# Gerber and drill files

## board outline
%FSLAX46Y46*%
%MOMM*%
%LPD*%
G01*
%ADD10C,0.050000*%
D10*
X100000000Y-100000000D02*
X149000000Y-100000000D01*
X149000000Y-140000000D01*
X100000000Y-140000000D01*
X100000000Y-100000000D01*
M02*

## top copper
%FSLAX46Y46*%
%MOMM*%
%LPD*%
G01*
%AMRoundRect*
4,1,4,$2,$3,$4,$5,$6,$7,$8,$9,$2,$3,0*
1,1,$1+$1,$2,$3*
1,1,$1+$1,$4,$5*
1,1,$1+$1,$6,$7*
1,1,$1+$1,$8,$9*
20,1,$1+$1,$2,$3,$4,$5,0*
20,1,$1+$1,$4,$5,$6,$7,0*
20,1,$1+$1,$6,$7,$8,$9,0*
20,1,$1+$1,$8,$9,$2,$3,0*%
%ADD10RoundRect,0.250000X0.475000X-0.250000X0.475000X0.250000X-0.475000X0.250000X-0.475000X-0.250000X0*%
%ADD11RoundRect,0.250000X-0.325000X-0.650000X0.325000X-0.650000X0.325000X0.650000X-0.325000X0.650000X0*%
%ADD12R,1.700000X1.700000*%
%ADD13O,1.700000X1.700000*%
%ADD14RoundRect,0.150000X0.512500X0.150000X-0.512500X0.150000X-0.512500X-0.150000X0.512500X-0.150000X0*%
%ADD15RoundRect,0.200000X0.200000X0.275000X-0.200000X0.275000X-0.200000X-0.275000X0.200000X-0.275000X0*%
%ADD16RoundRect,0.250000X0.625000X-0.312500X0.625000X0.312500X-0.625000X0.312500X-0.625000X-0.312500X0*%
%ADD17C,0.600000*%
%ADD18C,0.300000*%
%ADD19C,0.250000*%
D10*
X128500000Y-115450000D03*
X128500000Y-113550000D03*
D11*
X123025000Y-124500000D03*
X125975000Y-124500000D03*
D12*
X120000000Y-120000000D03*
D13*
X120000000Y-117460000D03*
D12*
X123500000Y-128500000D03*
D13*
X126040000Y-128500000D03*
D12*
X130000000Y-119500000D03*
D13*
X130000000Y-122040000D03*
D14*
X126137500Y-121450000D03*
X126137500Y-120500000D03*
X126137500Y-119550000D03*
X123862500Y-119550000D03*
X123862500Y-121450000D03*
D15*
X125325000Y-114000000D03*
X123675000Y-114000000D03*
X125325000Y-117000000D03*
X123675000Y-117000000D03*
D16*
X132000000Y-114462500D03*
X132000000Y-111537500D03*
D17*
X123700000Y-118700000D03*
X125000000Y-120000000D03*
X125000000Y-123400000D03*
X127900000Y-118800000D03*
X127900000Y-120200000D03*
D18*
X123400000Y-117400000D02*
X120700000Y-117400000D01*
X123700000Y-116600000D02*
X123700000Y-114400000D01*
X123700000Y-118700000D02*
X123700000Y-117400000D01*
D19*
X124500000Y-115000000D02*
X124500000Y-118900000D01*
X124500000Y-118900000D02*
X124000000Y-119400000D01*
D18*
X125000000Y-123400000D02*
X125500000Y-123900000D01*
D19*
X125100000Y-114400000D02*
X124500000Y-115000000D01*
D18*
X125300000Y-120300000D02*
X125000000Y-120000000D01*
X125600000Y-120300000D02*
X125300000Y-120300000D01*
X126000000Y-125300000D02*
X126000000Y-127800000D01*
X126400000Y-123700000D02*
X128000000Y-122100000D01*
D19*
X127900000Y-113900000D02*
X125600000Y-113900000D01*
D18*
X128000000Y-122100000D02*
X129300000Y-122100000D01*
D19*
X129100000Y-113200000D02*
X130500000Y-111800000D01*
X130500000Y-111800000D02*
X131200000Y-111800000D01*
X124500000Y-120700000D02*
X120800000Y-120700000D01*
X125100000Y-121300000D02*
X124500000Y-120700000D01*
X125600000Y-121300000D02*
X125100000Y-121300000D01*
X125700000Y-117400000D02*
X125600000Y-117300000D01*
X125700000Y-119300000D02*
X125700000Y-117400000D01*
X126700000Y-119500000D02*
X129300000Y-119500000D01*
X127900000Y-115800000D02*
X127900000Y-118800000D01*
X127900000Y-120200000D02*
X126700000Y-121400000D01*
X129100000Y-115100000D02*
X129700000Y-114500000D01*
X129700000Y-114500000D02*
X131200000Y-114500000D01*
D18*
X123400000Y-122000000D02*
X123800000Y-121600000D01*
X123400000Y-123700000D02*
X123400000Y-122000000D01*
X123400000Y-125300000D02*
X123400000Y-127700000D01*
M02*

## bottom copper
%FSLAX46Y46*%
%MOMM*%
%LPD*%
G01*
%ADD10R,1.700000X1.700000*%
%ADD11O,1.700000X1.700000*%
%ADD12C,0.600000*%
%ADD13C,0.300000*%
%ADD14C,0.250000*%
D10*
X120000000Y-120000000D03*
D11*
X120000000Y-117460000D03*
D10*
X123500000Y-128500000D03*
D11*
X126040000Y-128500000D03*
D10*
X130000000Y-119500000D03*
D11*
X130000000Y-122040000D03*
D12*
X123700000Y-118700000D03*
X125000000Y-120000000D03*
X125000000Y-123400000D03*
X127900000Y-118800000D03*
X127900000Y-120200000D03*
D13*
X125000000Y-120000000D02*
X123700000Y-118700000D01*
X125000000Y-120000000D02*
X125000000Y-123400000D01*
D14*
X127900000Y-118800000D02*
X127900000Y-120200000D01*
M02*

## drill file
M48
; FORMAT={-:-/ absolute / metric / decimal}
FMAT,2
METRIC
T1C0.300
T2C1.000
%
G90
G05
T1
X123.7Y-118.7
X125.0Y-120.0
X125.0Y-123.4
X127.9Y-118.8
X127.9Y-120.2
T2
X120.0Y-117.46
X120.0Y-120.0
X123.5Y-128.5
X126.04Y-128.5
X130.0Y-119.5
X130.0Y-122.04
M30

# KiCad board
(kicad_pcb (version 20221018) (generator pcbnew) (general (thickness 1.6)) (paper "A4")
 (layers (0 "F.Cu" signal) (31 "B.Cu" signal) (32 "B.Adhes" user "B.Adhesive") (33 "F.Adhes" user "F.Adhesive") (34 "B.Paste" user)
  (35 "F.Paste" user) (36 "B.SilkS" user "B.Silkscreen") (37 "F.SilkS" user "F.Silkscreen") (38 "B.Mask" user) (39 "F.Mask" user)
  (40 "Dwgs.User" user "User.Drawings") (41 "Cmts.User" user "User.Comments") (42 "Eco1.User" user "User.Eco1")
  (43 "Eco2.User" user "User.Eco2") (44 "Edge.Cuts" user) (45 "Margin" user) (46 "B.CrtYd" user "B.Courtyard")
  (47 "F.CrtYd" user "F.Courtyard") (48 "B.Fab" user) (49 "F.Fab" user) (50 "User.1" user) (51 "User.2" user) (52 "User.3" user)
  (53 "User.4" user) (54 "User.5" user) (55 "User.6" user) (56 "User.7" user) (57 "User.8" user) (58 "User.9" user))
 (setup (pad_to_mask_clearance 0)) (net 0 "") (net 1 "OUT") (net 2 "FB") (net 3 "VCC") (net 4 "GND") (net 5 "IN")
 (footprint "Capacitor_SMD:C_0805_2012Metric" (layer "F.Cu") (at 128.5 114.5 90)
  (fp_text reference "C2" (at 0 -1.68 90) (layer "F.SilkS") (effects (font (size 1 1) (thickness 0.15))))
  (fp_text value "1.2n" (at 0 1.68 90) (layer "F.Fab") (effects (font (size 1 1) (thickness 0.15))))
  (pad "1" smd roundrect (at -0.95 0 90) (size 1 1.45) (layers "F.Cu" "F.Paste" "F.Mask") (roundrect_rratio 0.25) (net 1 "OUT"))
  (pad "2" smd roundrect (at 0.95 0 90) (size 1 1.45) (layers "F.Cu" "F.Paste" "F.Mask") (roundrect_rratio 0.25) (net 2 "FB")))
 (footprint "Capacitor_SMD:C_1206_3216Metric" (layer "F.Cu") (at 124.5 124.5)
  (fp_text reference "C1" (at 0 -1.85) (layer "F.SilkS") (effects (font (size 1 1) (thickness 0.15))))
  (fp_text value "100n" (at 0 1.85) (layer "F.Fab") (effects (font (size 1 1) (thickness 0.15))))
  (pad "1" smd roundrect (at -1.475 0) (size 1.15 1.8) (layers "F.Cu" "F.Paste" "F.Mask") (roundrect_rratio 0.217391) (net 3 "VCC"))
  (pad "2" smd roundrect (at 1.475 0) (size 1.15 1.8) (layers "F.Cu" "F.Paste" "F.Mask") (roundrect_rratio 0.217391) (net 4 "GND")))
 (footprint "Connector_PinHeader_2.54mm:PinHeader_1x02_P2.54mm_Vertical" (layer "F.Cu") (at 120 120 180)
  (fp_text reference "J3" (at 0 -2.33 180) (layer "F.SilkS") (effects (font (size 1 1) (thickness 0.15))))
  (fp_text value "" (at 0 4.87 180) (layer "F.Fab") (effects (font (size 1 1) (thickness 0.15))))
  (pad "1" thru_hole rect (at 0 0 180) (size 1.7 1.7) (drill 1) (layers "*.Cu" "*.Mask") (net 1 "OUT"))
  (pad "2" thru_hole oval (at 0 2.54 180) (size 1.7 1.7) (drill 1) (layers "*.Cu" "*.Mask") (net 4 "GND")))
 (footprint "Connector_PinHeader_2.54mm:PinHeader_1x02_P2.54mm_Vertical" (layer "F.Cu") (at 123.5 128.5 90)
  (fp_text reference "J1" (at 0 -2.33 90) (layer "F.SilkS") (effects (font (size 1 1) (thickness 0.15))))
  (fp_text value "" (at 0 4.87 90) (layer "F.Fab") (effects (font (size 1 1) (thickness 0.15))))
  (pad "1" thru_hole rect (at 0 0 90) (size 1.7 1.7) (drill 1) (layers "*.Cu" "*.Mask") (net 3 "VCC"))
  (pad "2" thru_hole oval (at 0 2.54 90) (size 1.7 1.7) (drill 1) (layers "*.Cu" "*.Mask") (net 4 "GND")))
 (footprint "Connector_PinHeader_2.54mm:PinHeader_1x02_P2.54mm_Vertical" (layer "F.Cu") (at 130 119.5)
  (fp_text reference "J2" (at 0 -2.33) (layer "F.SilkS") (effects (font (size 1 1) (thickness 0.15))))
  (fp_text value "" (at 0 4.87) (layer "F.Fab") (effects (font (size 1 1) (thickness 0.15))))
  (pad "1" thru_hole rect (at 0 0) (size 1.7 1.7) (drill 1) (layers "*.Cu" "*.Mask") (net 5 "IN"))
  (pad "2" thru_hole oval (at 0 2.54) (size 1.7 1.7) (drill 1) (layers "*.Cu" "*.Mask") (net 4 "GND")))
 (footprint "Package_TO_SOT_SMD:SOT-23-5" (layer "F.Cu") (at 125 120.5 180)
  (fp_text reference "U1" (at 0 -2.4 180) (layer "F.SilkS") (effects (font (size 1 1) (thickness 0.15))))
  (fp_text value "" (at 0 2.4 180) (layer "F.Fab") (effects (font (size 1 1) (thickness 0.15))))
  (pad "1" smd roundrect (at -1.1375 -0.95 180) (size 1.325 0.6) (layers "F.Cu" "F.Paste" "F.Mask") (roundrect_rratio 0.25) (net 1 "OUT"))
  (pad "2" smd roundrect (at -1.1375 0 180) (size 1.325 0.6) (layers "F.Cu" "F.Paste" "F.Mask") (roundrect_rratio 0.25) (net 4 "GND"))
  (pad "3" smd roundrect (at -1.1375 0.95 180) (size 1.325 0.6) (layers "F.Cu" "F.Paste" "F.Mask") (roundrect_rratio 0.25) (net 5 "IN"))
  (pad "4" smd roundrect (at 1.1375 0.95 180) (size 1.325 0.6) (layers "F.Cu" "F.Paste" "F.Mask") (roundrect_rratio 0.25) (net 2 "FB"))
  (pad "5" smd roundrect (at 1.1375 -0.95 180) (size 1.325 0.6) (layers "F.Cu" "F.Paste" "F.Mask") (roundrect_rratio 0.25) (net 3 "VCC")))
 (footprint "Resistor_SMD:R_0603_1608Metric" (layer "F.Cu") (at 124.5 114 180)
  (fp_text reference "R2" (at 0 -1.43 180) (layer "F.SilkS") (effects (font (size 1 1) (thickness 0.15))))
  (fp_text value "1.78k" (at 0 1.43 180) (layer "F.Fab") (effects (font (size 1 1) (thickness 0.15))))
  (pad "1" smd roundrect (at -0.825 0 180) (size 0.8 0.95) (layers "F.Cu" "F.Paste" "F.Mask") (roundrect_rratio 0.25) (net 2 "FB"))
  (pad "2" smd roundrect (at 0.825 0 180) (size 0.8 0.95) (layers "F.Cu" "F.Paste" "F.Mask") (roundrect_rratio 0.25) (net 4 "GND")))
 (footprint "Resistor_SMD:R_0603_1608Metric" (layer "F.Cu") (at 124.5 117 180)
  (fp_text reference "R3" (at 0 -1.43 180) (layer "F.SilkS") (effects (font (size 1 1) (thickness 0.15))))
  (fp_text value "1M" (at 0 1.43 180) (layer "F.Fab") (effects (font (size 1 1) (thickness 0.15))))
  (pad "1" smd roundrect (at -0.825 0 180) (size 0.8 0.95) (layers "F.Cu" "F.Paste" "F.Mask") (roundrect_rratio 0.25) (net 5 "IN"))
  (pad "2" smd roundrect (at 0.825 0 180) (size 0.8 0.95) (layers "F.Cu" "F.Paste" "F.Mask") (roundrect_rratio 0.25) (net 4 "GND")))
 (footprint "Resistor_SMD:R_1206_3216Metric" (layer "F.Cu") (at 132 113 90)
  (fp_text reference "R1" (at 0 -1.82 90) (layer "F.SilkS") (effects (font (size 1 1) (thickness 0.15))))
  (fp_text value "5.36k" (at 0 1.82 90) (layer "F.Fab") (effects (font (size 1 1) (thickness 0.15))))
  (pad "1" smd roundrect (at -1.4625 0 90) (size 1.125 1.75) (layers "F.Cu" "F.Paste" "F.Mask") (roundrect_rratio 0.222222) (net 1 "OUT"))
  (pad "2" smd roundrect (at 1.4625 0 90) (size 1.125 1.75) (layers "F.Cu" "F.Paste" "F.Mask") (roundrect_rratio 0.222222) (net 2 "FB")))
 (gr_rect (start 100 100) (end 149 140) (stroke (width 0.05) (type default)) (fill none) (layer "Edge.Cuts"))
 (segment (start 123.4 117.4) (end 120.7 117.4) (width 0.3) (layer "F.Cu") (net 4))
 (segment (start 123.7 116.6) (end 123.7 114.4) (width 0.3) (layer "F.Cu") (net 4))
 (segment (start 123.7 118.7) (end 123.7 117.4) (width 0.3) (layer "F.Cu") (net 4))
 (segment (start 124.5 115) (end 124.5 118.9) (width 0.25) (layer "F.Cu") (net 2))
 (segment (start 124.5 118.9) (end 124 119.4) (width 0.25) (layer "F.Cu") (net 2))
 (segment (start 125 123.4) (end 125.5 123.9) (width 0.3) (layer "F.Cu") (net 4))
 (segment (start 125.1 114.4) (end 124.5 115) (width 0.25) (layer "F.Cu") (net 2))
 (segment (start 125.3 120.3) (end 125 120) (width 0.3) (layer "F.Cu") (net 4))
 (segment (start 125.6 120.3) (end 125.3 120.3) (width 0.3) (layer "F.Cu") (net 4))
 (segment (start 126 125.3) (end 126 127.8) (width 0.3) (layer "F.Cu") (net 4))
 (segment (start 126.4 123.7) (end 128 122.1) (width 0.3) (layer "F.Cu") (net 4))
 (segment (start 127.9 113.9) (end 125.6 113.9) (width 0.25) (layer "F.Cu") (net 2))
 (segment (start 128 122.1) (end 129.3 122.1) (width 0.3) (layer "F.Cu") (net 4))
 (segment (start 129.1 113.2) (end 130.5 111.8) (width 0.25) (layer "F.Cu") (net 2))
 (segment (start 130.5 111.8) (end 131.2 111.8) (width 0.25) (layer "F.Cu") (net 2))
 (via (at 123.7 118.7) (size 0.6) (drill 0.3) (layers "F.Cu" "B.Cu") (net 4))
 (via (at 125 120) (size 0.6) (drill 0.3) (layers "F.Cu" "B.Cu") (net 4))
 (via (at 125 123.4) (size 0.6) (drill 0.3) (layers "F.Cu" "B.Cu") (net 4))
 (segment (start 124.5 120.7) (end 120.8 120.7) (width 0.25) (layer "F.Cu") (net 1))
 (segment (start 125 120) (end 123.7 118.7) (width 0.3) (layer "B.Cu") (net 4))
 (segment (start 125 120) (end 125 123.4) (width 0.3) (layer "B.Cu") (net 4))
 (segment (start 125.1 121.3) (end 124.5 120.7) (width 0.25) (layer "F.Cu") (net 1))
 (segment (start 125.6 121.3) (end 125.1 121.3) (width 0.25) (layer "F.Cu") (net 1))
 (segment (start 125.7 117.4) (end 125.6 117.3) (width 0.25) (layer "F.Cu") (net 5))
 (segment (start 125.7 119.3) (end 125.7 117.4) (width 0.25) (layer "F.Cu") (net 5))
 (segment (start 126.7 119.5) (end 129.3 119.5) (width 0.25) (layer "F.Cu") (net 5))
 (segment (start 127.9 115.8) (end 127.9 118.8) (width 0.25) (layer "F.Cu") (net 1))
 (segment (start 127.9 120.2) (end 126.7 121.4) (width 0.25) (layer "F.Cu") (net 1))
 (segment (start 129.1 115.1) (end 129.7 114.5) (width 0.25) (layer "F.Cu") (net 1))
 (segment (start 129.7 114.5) (end 131.2 114.5) (width 0.25) (layer "F.Cu") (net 1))
 (via (at 127.9 118.8) (size 0.6) (drill 0.3) (layers "F.Cu" "B.Cu") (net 1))
 (via (at 127.9 120.2) (size 0.6) (drill 0.3) (layers "F.Cu" "B.Cu") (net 1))
 (segment (start 123.4 122) (end 123.8 121.6) (width 0.3) (layer "F.Cu") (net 3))
 (segment (start 123.4 123.7) (end 123.4 122) (width 0.3) (layer "F.Cu") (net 3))
 (segment (start 123.4 125.3) (end 123.4 127.7) (width 0.3) (layer "F.Cu") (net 3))
 (segment (start 127.9 118.8) (end 127.9 120.2) (width 0.25) (layer "B.Cu") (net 1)))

